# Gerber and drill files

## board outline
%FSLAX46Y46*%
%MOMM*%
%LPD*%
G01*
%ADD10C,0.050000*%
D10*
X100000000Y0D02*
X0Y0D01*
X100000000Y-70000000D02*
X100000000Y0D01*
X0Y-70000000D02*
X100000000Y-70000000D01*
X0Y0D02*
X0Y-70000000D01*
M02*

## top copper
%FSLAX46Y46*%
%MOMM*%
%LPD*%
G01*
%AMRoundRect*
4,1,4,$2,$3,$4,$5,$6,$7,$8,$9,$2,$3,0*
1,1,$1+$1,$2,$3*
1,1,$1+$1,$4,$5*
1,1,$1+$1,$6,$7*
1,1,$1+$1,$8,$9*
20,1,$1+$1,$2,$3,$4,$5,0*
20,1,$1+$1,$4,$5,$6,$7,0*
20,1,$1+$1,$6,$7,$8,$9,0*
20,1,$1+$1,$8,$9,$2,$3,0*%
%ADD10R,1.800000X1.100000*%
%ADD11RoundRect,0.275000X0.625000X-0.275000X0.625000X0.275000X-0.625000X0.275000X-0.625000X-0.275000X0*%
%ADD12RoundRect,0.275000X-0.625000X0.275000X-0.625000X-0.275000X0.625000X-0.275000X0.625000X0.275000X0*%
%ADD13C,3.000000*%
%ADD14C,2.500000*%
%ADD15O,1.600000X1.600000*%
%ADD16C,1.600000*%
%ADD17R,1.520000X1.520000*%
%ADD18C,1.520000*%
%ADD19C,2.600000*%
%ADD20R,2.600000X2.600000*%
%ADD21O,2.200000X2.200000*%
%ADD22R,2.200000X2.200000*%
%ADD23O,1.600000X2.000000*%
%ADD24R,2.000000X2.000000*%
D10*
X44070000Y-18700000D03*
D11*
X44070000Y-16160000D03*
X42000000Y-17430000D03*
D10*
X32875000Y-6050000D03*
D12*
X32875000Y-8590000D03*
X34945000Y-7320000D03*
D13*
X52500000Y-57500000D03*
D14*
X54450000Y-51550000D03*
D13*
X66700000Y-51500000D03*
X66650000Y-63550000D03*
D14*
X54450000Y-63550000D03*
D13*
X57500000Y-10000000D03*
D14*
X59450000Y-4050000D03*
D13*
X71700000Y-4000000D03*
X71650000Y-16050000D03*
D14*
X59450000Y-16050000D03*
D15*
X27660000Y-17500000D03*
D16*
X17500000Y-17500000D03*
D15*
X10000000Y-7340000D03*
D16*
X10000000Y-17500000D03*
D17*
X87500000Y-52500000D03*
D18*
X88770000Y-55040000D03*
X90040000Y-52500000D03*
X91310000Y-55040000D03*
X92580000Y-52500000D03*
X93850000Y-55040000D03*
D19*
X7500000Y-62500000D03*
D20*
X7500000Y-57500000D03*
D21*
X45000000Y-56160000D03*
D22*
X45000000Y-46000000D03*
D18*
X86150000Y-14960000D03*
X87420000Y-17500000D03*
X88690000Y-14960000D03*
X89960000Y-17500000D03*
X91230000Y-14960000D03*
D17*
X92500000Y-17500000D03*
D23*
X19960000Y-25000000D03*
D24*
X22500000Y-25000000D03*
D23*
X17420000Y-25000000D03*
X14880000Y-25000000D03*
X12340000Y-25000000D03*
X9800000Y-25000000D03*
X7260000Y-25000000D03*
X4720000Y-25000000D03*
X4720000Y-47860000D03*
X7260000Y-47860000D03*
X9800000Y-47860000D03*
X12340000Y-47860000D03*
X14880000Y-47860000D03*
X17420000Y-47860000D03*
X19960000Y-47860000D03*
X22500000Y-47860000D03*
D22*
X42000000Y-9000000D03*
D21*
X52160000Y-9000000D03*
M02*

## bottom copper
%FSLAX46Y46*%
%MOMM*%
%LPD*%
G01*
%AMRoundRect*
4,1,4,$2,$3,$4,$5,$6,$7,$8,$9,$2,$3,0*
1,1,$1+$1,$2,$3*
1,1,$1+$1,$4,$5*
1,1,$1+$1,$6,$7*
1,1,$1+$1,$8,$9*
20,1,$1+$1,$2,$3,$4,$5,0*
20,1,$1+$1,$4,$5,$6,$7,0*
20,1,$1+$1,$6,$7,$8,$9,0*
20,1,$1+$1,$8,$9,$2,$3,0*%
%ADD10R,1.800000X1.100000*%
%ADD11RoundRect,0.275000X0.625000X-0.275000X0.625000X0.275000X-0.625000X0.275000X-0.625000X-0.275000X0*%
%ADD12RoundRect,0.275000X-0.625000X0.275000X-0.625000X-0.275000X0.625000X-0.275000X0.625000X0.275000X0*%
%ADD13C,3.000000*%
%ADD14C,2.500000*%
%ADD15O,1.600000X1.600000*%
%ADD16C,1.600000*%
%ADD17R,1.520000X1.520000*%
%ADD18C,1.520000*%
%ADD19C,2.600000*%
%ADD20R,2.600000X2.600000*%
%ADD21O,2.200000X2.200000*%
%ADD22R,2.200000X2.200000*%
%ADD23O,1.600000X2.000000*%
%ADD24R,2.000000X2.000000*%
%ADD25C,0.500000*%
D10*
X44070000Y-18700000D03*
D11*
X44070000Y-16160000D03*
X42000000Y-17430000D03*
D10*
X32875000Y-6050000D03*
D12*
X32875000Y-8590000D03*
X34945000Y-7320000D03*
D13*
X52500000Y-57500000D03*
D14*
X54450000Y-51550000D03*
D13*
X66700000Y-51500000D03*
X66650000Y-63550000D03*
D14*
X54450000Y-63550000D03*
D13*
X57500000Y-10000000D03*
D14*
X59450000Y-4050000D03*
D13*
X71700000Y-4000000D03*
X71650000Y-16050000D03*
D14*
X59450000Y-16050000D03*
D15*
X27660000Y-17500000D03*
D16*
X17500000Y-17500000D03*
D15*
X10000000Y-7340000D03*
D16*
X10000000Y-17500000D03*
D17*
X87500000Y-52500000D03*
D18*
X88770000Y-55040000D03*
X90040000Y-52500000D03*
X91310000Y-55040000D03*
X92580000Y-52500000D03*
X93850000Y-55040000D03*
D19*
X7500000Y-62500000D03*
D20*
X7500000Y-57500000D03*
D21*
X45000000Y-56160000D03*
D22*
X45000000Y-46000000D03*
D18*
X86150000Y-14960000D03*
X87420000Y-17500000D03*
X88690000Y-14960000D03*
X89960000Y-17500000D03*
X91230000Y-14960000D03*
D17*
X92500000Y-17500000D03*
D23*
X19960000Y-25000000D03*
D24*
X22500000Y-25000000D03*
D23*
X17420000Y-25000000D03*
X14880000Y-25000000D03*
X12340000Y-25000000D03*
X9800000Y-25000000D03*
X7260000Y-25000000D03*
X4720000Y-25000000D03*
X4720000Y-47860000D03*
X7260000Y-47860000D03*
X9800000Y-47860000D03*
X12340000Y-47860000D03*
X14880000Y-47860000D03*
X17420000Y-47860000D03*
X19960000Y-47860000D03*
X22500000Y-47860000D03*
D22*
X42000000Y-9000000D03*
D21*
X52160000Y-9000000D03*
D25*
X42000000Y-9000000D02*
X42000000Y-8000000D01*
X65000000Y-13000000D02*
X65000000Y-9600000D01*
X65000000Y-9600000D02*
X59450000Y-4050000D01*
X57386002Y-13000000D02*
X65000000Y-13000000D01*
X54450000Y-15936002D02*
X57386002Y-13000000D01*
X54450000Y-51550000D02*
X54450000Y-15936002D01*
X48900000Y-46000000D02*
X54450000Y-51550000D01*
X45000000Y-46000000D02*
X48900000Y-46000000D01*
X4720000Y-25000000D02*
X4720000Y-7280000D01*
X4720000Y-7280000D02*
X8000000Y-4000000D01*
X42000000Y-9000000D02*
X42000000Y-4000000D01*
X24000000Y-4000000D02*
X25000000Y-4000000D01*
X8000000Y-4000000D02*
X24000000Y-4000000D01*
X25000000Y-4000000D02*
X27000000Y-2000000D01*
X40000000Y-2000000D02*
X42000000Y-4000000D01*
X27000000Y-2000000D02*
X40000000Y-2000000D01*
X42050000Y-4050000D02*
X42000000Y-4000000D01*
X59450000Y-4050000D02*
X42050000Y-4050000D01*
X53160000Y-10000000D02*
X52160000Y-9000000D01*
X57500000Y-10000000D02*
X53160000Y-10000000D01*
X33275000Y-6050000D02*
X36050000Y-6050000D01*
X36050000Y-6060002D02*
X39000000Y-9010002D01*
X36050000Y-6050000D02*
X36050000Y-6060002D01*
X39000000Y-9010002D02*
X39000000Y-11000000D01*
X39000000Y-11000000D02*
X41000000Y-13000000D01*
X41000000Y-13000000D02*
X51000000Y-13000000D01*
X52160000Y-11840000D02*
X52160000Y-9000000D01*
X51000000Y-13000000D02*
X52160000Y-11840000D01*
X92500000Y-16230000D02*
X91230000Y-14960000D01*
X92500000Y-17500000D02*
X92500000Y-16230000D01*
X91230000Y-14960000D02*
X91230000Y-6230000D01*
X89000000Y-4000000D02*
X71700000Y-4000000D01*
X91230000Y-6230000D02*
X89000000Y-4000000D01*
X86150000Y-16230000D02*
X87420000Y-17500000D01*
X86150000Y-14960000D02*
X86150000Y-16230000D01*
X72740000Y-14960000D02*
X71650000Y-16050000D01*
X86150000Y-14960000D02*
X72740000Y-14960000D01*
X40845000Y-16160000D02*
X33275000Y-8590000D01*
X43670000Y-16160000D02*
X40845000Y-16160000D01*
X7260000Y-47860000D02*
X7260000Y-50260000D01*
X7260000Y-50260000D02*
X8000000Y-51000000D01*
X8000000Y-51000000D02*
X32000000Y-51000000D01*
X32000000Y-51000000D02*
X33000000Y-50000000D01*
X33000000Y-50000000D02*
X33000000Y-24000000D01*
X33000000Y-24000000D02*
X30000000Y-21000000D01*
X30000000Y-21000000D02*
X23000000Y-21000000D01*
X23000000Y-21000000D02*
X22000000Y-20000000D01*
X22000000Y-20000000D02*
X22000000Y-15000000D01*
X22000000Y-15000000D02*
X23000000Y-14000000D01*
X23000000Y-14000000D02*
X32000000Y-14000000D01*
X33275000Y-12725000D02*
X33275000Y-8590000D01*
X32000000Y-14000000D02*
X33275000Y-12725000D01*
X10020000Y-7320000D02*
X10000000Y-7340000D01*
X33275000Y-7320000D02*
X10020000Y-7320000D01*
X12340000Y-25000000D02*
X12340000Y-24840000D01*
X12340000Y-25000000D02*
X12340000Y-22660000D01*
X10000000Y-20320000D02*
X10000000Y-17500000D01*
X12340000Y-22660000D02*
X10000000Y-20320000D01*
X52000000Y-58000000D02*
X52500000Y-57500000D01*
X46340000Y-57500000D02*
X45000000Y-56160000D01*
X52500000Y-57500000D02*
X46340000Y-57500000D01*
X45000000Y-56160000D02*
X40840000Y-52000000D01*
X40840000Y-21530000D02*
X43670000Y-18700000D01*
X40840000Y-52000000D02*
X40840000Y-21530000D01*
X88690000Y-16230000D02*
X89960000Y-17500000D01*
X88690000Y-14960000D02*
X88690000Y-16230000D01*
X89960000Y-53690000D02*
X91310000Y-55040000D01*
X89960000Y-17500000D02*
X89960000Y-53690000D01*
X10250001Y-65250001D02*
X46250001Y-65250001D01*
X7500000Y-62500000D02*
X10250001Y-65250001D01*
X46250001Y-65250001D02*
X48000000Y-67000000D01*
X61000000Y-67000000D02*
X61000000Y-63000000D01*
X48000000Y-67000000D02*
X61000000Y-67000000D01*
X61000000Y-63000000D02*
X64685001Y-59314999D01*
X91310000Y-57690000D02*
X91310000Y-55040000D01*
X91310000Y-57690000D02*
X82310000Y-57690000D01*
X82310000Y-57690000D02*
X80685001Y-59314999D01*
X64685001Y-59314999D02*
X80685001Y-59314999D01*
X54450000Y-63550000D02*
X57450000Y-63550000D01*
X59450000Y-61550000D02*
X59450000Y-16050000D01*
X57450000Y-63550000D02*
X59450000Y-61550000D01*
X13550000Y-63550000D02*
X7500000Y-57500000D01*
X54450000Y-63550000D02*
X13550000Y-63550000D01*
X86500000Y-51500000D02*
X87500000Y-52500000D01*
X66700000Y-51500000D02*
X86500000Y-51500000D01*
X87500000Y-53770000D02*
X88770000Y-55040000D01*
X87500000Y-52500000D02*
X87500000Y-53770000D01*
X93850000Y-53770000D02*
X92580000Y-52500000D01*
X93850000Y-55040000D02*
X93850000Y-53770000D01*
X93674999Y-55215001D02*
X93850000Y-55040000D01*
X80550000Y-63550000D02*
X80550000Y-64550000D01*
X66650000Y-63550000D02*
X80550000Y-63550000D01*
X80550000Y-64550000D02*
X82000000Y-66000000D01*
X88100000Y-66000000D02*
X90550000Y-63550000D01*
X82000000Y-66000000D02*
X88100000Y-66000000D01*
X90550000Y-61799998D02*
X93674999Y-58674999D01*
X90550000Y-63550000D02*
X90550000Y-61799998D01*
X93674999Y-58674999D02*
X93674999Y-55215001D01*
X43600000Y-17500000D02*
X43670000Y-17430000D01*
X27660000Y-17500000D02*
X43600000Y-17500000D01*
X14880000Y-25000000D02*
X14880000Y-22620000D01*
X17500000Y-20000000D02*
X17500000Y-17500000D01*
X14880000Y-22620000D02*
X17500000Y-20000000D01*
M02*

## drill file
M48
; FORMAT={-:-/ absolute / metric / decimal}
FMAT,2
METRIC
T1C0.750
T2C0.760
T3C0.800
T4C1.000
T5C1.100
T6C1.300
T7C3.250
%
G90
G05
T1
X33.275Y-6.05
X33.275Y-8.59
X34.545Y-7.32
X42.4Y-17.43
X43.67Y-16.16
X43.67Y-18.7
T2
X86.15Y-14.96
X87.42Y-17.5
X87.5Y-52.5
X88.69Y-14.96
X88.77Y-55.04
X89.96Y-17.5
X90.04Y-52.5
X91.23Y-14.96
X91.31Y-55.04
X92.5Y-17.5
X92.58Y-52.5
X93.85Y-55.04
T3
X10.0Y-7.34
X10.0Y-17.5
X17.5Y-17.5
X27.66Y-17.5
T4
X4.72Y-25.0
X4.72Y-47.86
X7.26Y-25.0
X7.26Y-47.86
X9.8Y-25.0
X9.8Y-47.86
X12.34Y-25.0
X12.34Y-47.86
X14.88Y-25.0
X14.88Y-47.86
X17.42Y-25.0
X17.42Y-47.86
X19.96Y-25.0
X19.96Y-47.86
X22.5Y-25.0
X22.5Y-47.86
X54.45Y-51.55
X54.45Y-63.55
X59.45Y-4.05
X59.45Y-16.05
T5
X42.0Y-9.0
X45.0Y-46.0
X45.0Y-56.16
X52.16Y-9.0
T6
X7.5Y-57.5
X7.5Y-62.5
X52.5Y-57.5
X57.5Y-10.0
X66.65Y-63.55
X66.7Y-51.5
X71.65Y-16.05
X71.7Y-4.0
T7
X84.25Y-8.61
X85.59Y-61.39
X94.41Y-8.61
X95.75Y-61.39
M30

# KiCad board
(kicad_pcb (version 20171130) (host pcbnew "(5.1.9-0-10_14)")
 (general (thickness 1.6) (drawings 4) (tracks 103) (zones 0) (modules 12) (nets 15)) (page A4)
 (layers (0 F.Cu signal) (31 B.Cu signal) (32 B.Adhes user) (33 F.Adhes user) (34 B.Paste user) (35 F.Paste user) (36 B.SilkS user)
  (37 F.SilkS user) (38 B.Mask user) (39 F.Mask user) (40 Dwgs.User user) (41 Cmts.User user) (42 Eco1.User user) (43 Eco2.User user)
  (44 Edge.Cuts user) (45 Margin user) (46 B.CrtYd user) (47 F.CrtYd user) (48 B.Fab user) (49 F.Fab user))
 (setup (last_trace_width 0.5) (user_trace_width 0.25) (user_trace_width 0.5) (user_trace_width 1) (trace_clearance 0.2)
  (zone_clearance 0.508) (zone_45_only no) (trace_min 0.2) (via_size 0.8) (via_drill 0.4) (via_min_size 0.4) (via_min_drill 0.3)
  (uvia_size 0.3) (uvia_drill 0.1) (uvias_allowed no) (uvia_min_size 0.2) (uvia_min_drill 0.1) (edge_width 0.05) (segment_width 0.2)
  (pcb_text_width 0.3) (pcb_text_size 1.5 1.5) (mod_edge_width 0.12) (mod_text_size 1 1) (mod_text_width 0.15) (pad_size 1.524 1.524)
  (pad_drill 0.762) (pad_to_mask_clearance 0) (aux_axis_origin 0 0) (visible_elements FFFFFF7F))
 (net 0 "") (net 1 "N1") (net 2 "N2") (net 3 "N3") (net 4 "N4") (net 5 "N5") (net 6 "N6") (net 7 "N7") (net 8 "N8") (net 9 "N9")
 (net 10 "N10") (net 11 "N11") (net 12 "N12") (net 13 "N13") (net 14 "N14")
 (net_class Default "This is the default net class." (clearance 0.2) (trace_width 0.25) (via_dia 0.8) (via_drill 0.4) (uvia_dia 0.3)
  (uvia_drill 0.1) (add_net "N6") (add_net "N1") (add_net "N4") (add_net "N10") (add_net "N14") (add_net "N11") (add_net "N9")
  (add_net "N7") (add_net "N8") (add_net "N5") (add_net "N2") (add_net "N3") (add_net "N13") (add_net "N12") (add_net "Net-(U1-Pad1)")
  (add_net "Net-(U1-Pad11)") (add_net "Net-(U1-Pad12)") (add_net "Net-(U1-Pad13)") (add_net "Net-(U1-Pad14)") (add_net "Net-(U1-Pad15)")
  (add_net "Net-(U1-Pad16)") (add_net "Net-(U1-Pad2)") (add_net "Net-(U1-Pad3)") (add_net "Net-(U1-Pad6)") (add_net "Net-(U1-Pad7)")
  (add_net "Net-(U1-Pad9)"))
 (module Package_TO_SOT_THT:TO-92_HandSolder (layer F.Cu) (at 43.67 18.7 90)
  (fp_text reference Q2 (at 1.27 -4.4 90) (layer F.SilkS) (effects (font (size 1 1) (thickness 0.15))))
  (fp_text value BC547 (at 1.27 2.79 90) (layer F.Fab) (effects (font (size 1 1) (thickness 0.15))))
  (pad 1 thru_hole rect (at 0 0 90) (size 1.1 1.8) (drill 0.75 (offset 0 0.4)) (layers *.Cu *.Mask) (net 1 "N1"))
  (pad 3 thru_hole roundrect (at 2.54 0 90) (size 1.1 1.8) (drill 0.75 (offset 0 0.4)) (layers *.Cu *.Mask) (roundrect_rratio 0.25)
   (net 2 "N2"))
  (pad 2 thru_hole roundrect (at 1.27 -1.27 90) (size 1.1 1.8) (drill 0.75 (offset 0 -0.4)) (layers *.Cu *.Mask) (roundrect_rratio 0.25)
   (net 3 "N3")))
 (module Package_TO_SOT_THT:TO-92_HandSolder (layer F.Cu) (at 33.275 6.05 270)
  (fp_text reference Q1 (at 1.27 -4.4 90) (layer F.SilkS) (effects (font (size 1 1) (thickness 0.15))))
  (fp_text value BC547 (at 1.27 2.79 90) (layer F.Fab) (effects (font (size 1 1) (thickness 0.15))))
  (pad 1 thru_hole rect (at 0 0 270) (size 1.1 1.8) (drill 0.75 (offset 0 0.4)) (layers *.Cu *.Mask) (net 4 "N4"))
  (pad 3 thru_hole roundrect (at 2.54 0 270) (size 1.1 1.8) (drill 0.75 (offset 0 0.4)) (layers *.Cu *.Mask) (roundrect_rratio 0.25)
   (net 2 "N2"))
  (pad 2 thru_hole roundrect (at 1.27 -1.27 270) (size 1.1 1.8) (drill 0.75 (offset 0 -0.4)) (layers *.Cu *.Mask) (roundrect_rratio 0.25)
   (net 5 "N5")))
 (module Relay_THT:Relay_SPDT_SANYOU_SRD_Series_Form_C (layer F.Cu) (at 52.5 57.5)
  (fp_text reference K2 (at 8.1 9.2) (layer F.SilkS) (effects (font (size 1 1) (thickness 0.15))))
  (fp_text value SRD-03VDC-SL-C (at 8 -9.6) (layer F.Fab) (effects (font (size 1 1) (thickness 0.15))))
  (pad 1 thru_hole circle (at 0 0 90) (size 3 3) (drill 1.3) (layers *.Cu *.Mask) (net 1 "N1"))
  (pad 5 thru_hole circle (at 1.95 -5.95 90) (size 2.5 2.5) (drill 1) (layers *.Cu *.Mask) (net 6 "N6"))
  (pad 4 thru_hole circle (at 14.2 -6 90) (size 3 3) (drill 1.3) (layers *.Cu *.Mask) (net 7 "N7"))
  (pad 3 thru_hole circle (at 14.15 6.05 90) (size 3 3) (drill 1.3) (layers *.Cu *.Mask) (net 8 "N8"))
  (pad 2 thru_hole circle (at 1.95 6.05 90) (size 2.5 2.5) (drill 1) (layers *.Cu *.Mask) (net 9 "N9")))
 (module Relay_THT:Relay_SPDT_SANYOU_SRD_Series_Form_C (layer F.Cu) (at 57.5 10)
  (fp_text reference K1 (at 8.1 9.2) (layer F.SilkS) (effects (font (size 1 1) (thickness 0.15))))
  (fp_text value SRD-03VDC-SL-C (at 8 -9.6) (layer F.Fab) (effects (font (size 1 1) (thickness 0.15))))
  (pad 1 thru_hole circle (at 0 0 90) (size 3 3) (drill 1.3) (layers *.Cu *.Mask) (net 4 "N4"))
  (pad 5 thru_hole circle (at 1.95 -5.95 90) (size 2.5 2.5) (drill 1) (layers *.Cu *.Mask) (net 6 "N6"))
  (pad 4 thru_hole circle (at 14.2 -6 90) (size 3 3) (drill 1.3) (layers *.Cu *.Mask) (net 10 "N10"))
  (pad 3 thru_hole circle (at 14.15 6.05 90) (size 3 3) (drill 1.3) (layers *.Cu *.Mask) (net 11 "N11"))
  (pad 2 thru_hole circle (at 1.95 6.05 90) (size 2.5 2.5) (drill 1) (layers *.Cu *.Mask) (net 9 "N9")))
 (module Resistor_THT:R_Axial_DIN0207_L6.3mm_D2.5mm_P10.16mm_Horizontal (layer F.Cu) (at 17.5 17.5)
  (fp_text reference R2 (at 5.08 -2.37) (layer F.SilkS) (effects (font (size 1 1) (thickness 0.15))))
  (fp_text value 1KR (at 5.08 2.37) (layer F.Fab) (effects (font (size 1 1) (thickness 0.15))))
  (pad 2 thru_hole oval (at 10.16 0) (size 1.6 1.6) (drill 0.8) (layers *.Cu *.Mask) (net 3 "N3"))
  (pad 1 thru_hole circle (at 0 0) (size 1.6 1.6) (drill 0.8) (layers *.Cu *.Mask) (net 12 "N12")))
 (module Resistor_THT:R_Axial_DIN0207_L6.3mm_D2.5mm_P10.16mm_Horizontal (layer F.Cu) (at 10 17.5 90)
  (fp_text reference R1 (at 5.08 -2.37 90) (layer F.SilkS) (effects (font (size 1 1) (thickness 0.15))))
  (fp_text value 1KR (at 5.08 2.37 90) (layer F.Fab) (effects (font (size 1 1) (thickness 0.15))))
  (pad 2 thru_hole oval (at 10.16 0 90) (size 1.6 1.6) (drill 0.8) (layers *.Cu *.Mask) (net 5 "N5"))
  (pad 1 thru_hole circle (at 0 0 90) (size 1.6 1.6) (drill 0.8) (layers *.Cu *.Mask) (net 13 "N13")))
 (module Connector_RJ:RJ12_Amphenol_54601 (layer F.Cu) (at 87.5 52.5)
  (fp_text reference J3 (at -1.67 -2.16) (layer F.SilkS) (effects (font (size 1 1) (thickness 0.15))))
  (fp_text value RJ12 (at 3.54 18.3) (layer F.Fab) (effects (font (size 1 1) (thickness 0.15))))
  (pad 1 thru_hole rect (at 0 0) (size 1.52 1.52) (drill 0.76) (layers *.Cu *.Mask) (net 7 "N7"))
  (pad "" np_thru_hole circle (at -1.91 8.89) (size 3.25 3.25) (drill 3.25) (layers *.Cu *.Mask))
  (pad 2 thru_hole circle (at 1.27 2.54) (size 1.52 1.52) (drill 0.76) (layers *.Cu *.Mask) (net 7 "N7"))
  (pad 3 thru_hole circle (at 2.54 0) (size 1.52 1.52) (drill 0.76) (layers *.Cu *.Mask) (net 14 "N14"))
  (pad 4 thru_hole circle (at 3.81 2.54) (size 1.52 1.52) (drill 0.76) (layers *.Cu *.Mask) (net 14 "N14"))
  (pad 5 thru_hole circle (at 5.08 0) (size 1.52 1.52) (drill 0.76) (layers *.Cu *.Mask) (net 8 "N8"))
  (pad 6 thru_hole circle (at 6.35 2.54) (size 1.52 1.52) (drill 0.76) (layers *.Cu *.Mask) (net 8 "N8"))
  (pad "" np_thru_hole circle (at 8.25 8.89) (size 3.25 3.25) (drill 3.25) (layers *.Cu *.Mask)))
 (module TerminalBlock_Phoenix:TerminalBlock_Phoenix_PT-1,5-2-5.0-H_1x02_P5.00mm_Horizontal (layer F.Cu) (at 7.5 57.5 270)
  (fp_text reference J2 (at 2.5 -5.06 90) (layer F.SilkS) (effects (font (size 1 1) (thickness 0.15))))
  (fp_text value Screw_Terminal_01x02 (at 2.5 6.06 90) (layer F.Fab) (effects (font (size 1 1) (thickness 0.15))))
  (pad 2 thru_hole circle (at 5 0 270) (size 2.6 2.6) (drill 1.3) (layers *.Cu *.Mask) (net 14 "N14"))
  (pad 1 thru_hole rect (at 0 0 270) (size 2.6 2.6) (drill 1.3) (layers *.Cu *.Mask) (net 9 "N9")))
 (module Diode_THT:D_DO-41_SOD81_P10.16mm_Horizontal (layer F.Cu) (at 45 46 270)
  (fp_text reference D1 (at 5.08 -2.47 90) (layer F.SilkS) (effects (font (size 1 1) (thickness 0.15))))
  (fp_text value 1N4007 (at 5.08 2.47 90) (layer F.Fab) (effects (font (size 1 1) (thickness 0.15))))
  (pad 2 thru_hole oval (at 10.16 0 270) (size 2.2 2.2) (drill 1.1) (layers *.Cu *.Mask) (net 1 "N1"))
  (pad 1 thru_hole rect (at 0 0 270) (size 2.2 2.2) (drill 1.1) (layers *.Cu *.Mask) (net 6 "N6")))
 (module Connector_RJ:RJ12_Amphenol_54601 (layer F.Cu) (at 92.5 17.5 180)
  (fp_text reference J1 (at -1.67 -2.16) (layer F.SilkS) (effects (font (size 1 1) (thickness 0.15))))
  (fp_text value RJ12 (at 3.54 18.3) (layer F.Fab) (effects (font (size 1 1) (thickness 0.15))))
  (pad "" np_thru_hole circle (at 8.25 8.89 180) (size 3.25 3.25) (drill 3.25) (layers *.Cu *.Mask))
  (pad 6 thru_hole circle (at 6.35 2.54 180) (size 1.52 1.52) (drill 0.76) (layers *.Cu *.Mask) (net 11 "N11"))
  (pad 5 thru_hole circle (at 5.08 0 180) (size 1.52 1.52) (drill 0.76) (layers *.Cu *.Mask) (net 11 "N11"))
  (pad 4 thru_hole circle (at 3.81 2.54 180) (size 1.52 1.52) (drill 0.76) (layers *.Cu *.Mask) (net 14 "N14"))
  (pad 3 thru_hole circle (at 2.54 0 180) (size 1.52 1.52) (drill 0.76) (layers *.Cu *.Mask) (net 14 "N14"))
  (pad 2 thru_hole circle (at 1.27 2.54 180) (size 1.52 1.52) (drill 0.76) (layers *.Cu *.Mask) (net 10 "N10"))
  (pad "" np_thru_hole circle (at -1.91 8.89 180) (size 3.25 3.25) (drill 3.25) (layers *.Cu *.Mask))
  (pad 1 thru_hole rect (at 0 0 180) (size 1.52 1.52) (drill 0.76) (layers *.Cu *.Mask) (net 10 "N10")))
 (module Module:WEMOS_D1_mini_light (layer F.Cu) (at 22.5 25 270)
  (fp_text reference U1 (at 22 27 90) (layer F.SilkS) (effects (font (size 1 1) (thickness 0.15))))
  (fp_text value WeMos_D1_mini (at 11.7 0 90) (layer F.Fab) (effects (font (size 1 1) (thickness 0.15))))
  (pad 2 thru_hole oval (at 0 2.54 270) (size 2 1.6) (drill 1) (layers *.Cu *.Mask))
  (pad 1 thru_hole rect (at 0 0 270) (size 2 2) (drill 1) (layers *.Cu *.Mask))
  (pad 3 thru_hole oval (at 0 5.08 270) (size 2 1.6) (drill 1) (layers *.Cu *.Mask))
  (pad 4 thru_hole oval (at 0 7.62 270) (size 2 1.6) (drill 1) (layers *.Cu *.Mask) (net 12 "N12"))
  (pad 5 thru_hole oval (at 0 10.16 270) (size 2 1.6) (drill 1) (layers *.Cu *.Mask) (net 13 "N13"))
  (pad 6 thru_hole oval (at 0 12.7 270) (size 2 1.6) (drill 1) (layers *.Cu *.Mask))
  (pad 7 thru_hole oval (at 0 15.24 270) (size 2 1.6) (drill 1) (layers *.Cu *.Mask))
  (pad 8 thru_hole oval (at 0 17.78 270) (size 2 1.6) (drill 1) (layers *.Cu *.Mask) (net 6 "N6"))
  (pad 9 thru_hole oval (at 22.86 17.78 270) (size 2 1.6) (drill 1) (layers *.Cu *.Mask))
  (pad 10 thru_hole oval (at 22.86 15.24 270) (size 2 1.6) (drill 1) (layers *.Cu *.Mask) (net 2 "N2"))
  (pad 11 thru_hole oval (at 22.86 12.7 270) (size 2 1.6) (drill 1) (layers *.Cu *.Mask))
  (pad 12 thru_hole oval (at 22.86 10.16 270) (size 2 1.6) (drill 1) (layers *.Cu *.Mask))
  (pad 13 thru_hole oval (at 22.86 7.62 270) (size 2 1.6) (drill 1) (layers *.Cu *.Mask))
  (pad 14 thru_hole oval (at 22.86 5.08 270) (size 2 1.6) (drill 1) (layers *.Cu *.Mask))
  (pad 15 thru_hole oval (at 22.86 2.54 270) (size 2 1.6) (drill 1) (layers *.Cu *.Mask))
  (pad 16 thru_hole oval (at 22.86 0 270) (size 2 1.6) (drill 1) (layers *.Cu *.Mask)))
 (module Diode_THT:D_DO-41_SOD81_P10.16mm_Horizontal (layer F.Cu) (at 42 9)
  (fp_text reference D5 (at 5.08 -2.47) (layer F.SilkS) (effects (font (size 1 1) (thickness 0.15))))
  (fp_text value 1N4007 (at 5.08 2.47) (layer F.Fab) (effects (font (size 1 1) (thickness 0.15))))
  (pad 1 thru_hole rect (at 0 0) (size 2.2 2.2) (drill 1.1) (layers *.Cu *.Mask) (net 6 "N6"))
  (pad 2 thru_hole oval (at 10.16 0) (size 2.2 2.2) (drill 1.1) (layers *.Cu *.Mask) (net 4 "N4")))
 (gr_line (start 100 0) (end 0 0) (layer Edge.Cuts) (width 0.05))
 (gr_line (start 100 70) (end 100 0) (layer Edge.Cuts) (width 0.05))
 (gr_line (start 0 70) (end 100 70) (layer Edge.Cuts) (width 0.05))
 (gr_line (start 0 0) (end 0 70) (layer Edge.Cuts) (width 0.05))
 (segment (start 42 9) (end 42 8) (width 0.5) (layer B.Cu) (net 6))
 (segment (start 65 13) (end 65 9.6) (width 0.5) (layer B.Cu) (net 6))
 (segment (start 65 9.6) (end 59.45 4.05) (width 0.5) (layer B.Cu) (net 6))
 (segment (start 57.386002 13) (end 65 13) (width 0.5) (layer B.Cu) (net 6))
 (segment (start 54.45 15.936002) (end 57.386002 13) (width 0.5) (layer B.Cu) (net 6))
 (segment (start 54.45 51.55) (end 54.45 15.936002) (width 0.5) (layer B.Cu) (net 6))
 (segment (start 48.9 46) (end 54.45 51.55) (width 0.5) (layer B.Cu) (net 6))
 (segment (start 45 46) (end 48.9 46) (width 0.5) (layer B.Cu) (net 6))
 (segment (start 4.72 25) (end 4.72 7.28) (width 0.5) (layer B.Cu) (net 6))
 (segment (start 4.72 7.28) (end 8 4) (width 0.5) (layer B.Cu) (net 6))
 (segment (start 42 9) (end 42 4) (width 0.5) (layer B.Cu) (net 6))
 (segment (start 24 4) (end 25 4) (width 0.5) (layer B.Cu) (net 6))
 (segment (start 8 4) (end 24 4) (width 0.5) (layer B.Cu) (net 6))
 (segment (start 25 4) (end 27 2) (width 0.5) (layer B.Cu) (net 6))
 (segment (start 40 2) (end 42 4) (width 0.5) (layer B.Cu) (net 6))
 (segment (start 27 2) (end 40 2) (width 0.5) (layer B.Cu) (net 6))
 (segment (start 42.05 4.05) (end 42 4) (width 0.5) (layer B.Cu) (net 6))
 (segment (start 59.45 4.05) (end 42.05 4.05) (width 0.5) (layer B.Cu) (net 6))
 (segment (start 53.16 10) (end 52.16 9) (width 0.5) (layer B.Cu) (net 4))
 (segment (start 57.5 10) (end 53.16 10) (width 0.5) (layer B.Cu) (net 4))
 (segment (start 33.275 6.05) (end 36.05 6.05) (width 0.5) (layer B.Cu) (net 4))
 (segment (start 36.05 6.060002) (end 39 9.010002) (width 0.5) (layer B.Cu) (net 4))
 (segment (start 36.05 6.05) (end 36.05 6.060002) (width 0.5) (layer B.Cu) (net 4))
 (segment (start 39 9.010002) (end 39 11) (width 0.5) (layer B.Cu) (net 4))
 (segment (start 39 11) (end 41 13) (width 0.5) (layer B.Cu) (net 4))
 (segment (start 41 13) (end 51 13) (width 0.5) (layer B.Cu) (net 4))
 (segment (start 52.16 11.84) (end 52.16 9) (width 0.5) (layer B.Cu) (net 4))
 (segment (start 51 13) (end 52.16 11.84) (width 0.5) (layer B.Cu) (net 4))
 (segment (start 92.5 16.23) (end 91.23 14.96) (width 0.5) (layer B.Cu) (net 10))
 (segment (start 92.5 17.5) (end 92.5 16.23) (width 0.5) (layer B.Cu) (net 10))
 (segment (start 91.23 14.96) (end 91.23 6.23) (width 0.5) (layer B.Cu) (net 10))
 (segment (start 89 4) (end 71.7 4) (width 0.5) (layer B.Cu) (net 10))
 (segment (start 91.23 6.23) (end 89 4) (width 0.5) (layer B.Cu) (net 10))
 (segment (start 86.15 16.23) (end 87.42 17.5) (width 0.5) (layer B.Cu) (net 11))
 (segment (start 86.15 14.96) (end 86.15 16.23) (width 0.5) (layer B.Cu) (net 11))
 (segment (start 72.74 14.96) (end 71.65 16.05) (width 0.5) (layer B.Cu) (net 11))
 (segment (start 86.15 14.96) (end 72.74 14.96) (width 0.5) (layer B.Cu) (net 11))
 (segment (start 40.845 16.16) (end 33.275 8.59) (width 0.5) (layer B.Cu) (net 2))
 (segment (start 43.67 16.16) (end 40.845 16.16) (width 0.5) (layer B.Cu) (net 2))
 (segment (start 7.26 47.86) (end 7.26 50.26) (width 0.5) (layer B.Cu) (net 2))
 (segment (start 7.26 50.26) (end 8 51) (width 0.5) (layer B.Cu) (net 2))
 (segment (start 8 51) (end 32 51) (width 0.5) (layer B.Cu) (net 2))
 (segment (start 32 51) (end 33 50) (width 0.5) (layer B.Cu) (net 2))
 (segment (start 33 50) (end 33 24) (width 0.5) (layer B.Cu) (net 2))
 (segment (start 33 24) (end 30 21) (width 0.5) (layer B.Cu) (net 2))
 (segment (start 30 21) (end 23 21) (width 0.5) (layer B.Cu) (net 2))
 (segment (start 23 21) (end 22 20) (width 0.5) (layer B.Cu) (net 2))
 (segment (start 22 20) (end 22 15) (width 0.5) (layer B.Cu) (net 2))
 (segment (start 22 15) (end 23 14) (width 0.5) (layer B.Cu) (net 2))
 (segment (start 23 14) (end 32 14) (width 0.5) (layer B.Cu) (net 2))
 (segment (start 33.275 12.725) (end 33.275 8.59) (width 0.5) (layer B.Cu) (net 2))
 (segment (start 32 14) (end 33.275 12.725) (width 0.5) (layer B.Cu) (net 2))
 (segment (start 10.02 7.32) (end 10 7.34) (width 0.5) (layer B.Cu) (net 5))
 (segment (start 33.275 7.32) (end 10.02 7.32) (width 0.5) (layer B.Cu) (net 5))
 (segment (start 12.34 25) (end 12.34 24.84) (width 0.5) (layer B.Cu) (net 13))
 (segment (start 12.34 25) (end 12.34 22.66) (width 0.5) (layer B.Cu) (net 13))
 (segment (start 10 20.32) (end 10 17.5) (width 0.5) (layer B.Cu) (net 13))
 (segment (start 12.34 22.66) (end 10 20.32) (width 0.5) (layer B.Cu) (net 13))
 (segment (start 52 58) (end 52.5 57.5) (width 0.5) (layer B.Cu) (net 1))
 (segment (start 46.34 57.5) (end 45 56.16) (width 0.5) (layer B.Cu) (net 1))
 (segment (start 52.5 57.5) (end 46.34 57.5) (width 0.5) (layer B.Cu) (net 1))
 (segment (start 45 56.16) (end 40.84 52) (width 0.5) (layer B.Cu) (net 1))
 (segment (start 40.84 21.53) (end 43.67 18.7) (width 0.5) (layer B.Cu) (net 1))
 (segment (start 40.84 52) (end 40.84 21.53) (width 0.5) (layer B.Cu) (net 1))
 (segment (start 88.69 16.23) (end 89.96 17.5) (width 0.5) (layer B.Cu) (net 14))
 (segment (start 88.69 14.96) (end 88.69 16.23) (width 0.5) (layer B.Cu) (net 14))
 (segment (start 89.96 53.69) (end 91.31 55.04) (width 0.5) (layer B.Cu) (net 14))
 (segment (start 89.96 17.5) (end 89.96 53.69) (width 0.5) (layer B.Cu) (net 14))
 (segment (start 10.250001 65.250001) (end 46.250001 65.250001) (width 0.5) (layer B.Cu) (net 14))
 (segment (start 7.5 62.5) (end 10.250001 65.250001) (width 0.5) (layer B.Cu) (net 14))
 (segment (start 46.250001 65.250001) (end 48 67) (width 0.5) (layer B.Cu) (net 14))
 (segment (start 61 67) (end 61 63) (width 0.5) (layer B.Cu) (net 14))
 (segment (start 48 67) (end 61 67) (width 0.5) (layer B.Cu) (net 14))
 (segment (start 61 63) (end 64.685001 59.314999) (width 0.5) (layer B.Cu) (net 14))
 (segment (start 91.31 57.69) (end 91.31 55.04) (width 0.5) (layer B.Cu) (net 14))
 (segment (start 91.31 57.69) (end 82.31 57.69) (width 0.5) (layer B.Cu) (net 14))
 (segment (start 82.31 57.69) (end 80.685001 59.314999) (width 0.5) (layer B.Cu) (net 14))
 (segment (start 64.685001 59.314999) (end 80.685001 59.314999) (width 0.5) (layer B.Cu) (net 14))
 (segment (start 54.45 63.55) (end 57.45 63.55) (width 0.5) (layer B.Cu) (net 9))
 (segment (start 59.45 61.55) (end 59.45 16.05) (width 0.5) (layer B.Cu) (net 9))
 (segment (start 57.45 63.55) (end 59.45 61.55) (width 0.5) (layer B.Cu) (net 9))
 (segment (start 13.55 63.55) (end 7.5 57.5) (width 0.5) (layer B.Cu) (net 9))
 (segment (start 54.45 63.55) (end 13.55 63.55) (width 0.5) (layer B.Cu) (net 9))
 (segment (start 86.5 51.5) (end 87.5 52.5) (width 0.5) (layer B.Cu) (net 7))
 (segment (start 66.7 51.5) (end 86.5 51.5) (width 0.5) (layer B.Cu) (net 7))
 (segment (start 87.5 53.77) (end 88.77 55.04) (width 0.5) (layer B.Cu) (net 7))
 (segment (start 87.5 52.5) (end 87.5 53.77) (width 0.5) (layer B.Cu) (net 7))
 (segment (start 93.85 53.77) (end 92.58 52.5) (width 0.5) (layer B.Cu) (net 8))
 (segment (start 93.85 55.04) (end 93.85 53.77) (width 0.5) (layer B.Cu) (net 8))
 (segment (start 93.674999 55.215001) (end 93.85 55.04) (width 0.5) (layer B.Cu) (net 8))
 (segment (start 80.55 63.55) (end 80.55 64.55) (width 0.5) (layer B.Cu) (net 8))
 (segment (start 66.65 63.55) (end 80.55 63.55) (width 0.5) (layer B.Cu) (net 8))
 (segment (start 80.55 64.55) (end 82 66) (width 0.5) (layer B.Cu) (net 8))
 (segment (start 88.1 66) (end 90.55 63.55) (width 0.5) (layer B.Cu) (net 8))
 (segment (start 82 66) (end 88.1 66) (width 0.5) (layer B.Cu) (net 8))
 (segment (start 90.55 61.799998) (end 93.674999 58.674999) (width 0.5) (layer B.Cu) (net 8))
 (segment (start 90.55 63.55) (end 90.55 61.799998) (width 0.5) (layer B.Cu) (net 8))
 (segment (start 93.674999 58.674999) (end 93.674999 55.215001) (width 0.5) (layer B.Cu) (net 8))
 (segment (start 43.6 17.5) (end 43.67 17.43) (width 0.5) (layer B.Cu) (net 3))
 (segment (start 27.66 17.5) (end 43.6 17.5) (width 0.5) (layer B.Cu) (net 3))
 (segment (start 14.88 25) (end 14.88 22.62) (width 0.5) (layer B.Cu) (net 12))
 (segment (start 17.5 20) (end 17.5 17.5) (width 0.5) (layer B.Cu) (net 12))
 (segment (start 14.88 22.62) (end 17.5 20) (width 0.5) (layer B.Cu) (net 12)))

